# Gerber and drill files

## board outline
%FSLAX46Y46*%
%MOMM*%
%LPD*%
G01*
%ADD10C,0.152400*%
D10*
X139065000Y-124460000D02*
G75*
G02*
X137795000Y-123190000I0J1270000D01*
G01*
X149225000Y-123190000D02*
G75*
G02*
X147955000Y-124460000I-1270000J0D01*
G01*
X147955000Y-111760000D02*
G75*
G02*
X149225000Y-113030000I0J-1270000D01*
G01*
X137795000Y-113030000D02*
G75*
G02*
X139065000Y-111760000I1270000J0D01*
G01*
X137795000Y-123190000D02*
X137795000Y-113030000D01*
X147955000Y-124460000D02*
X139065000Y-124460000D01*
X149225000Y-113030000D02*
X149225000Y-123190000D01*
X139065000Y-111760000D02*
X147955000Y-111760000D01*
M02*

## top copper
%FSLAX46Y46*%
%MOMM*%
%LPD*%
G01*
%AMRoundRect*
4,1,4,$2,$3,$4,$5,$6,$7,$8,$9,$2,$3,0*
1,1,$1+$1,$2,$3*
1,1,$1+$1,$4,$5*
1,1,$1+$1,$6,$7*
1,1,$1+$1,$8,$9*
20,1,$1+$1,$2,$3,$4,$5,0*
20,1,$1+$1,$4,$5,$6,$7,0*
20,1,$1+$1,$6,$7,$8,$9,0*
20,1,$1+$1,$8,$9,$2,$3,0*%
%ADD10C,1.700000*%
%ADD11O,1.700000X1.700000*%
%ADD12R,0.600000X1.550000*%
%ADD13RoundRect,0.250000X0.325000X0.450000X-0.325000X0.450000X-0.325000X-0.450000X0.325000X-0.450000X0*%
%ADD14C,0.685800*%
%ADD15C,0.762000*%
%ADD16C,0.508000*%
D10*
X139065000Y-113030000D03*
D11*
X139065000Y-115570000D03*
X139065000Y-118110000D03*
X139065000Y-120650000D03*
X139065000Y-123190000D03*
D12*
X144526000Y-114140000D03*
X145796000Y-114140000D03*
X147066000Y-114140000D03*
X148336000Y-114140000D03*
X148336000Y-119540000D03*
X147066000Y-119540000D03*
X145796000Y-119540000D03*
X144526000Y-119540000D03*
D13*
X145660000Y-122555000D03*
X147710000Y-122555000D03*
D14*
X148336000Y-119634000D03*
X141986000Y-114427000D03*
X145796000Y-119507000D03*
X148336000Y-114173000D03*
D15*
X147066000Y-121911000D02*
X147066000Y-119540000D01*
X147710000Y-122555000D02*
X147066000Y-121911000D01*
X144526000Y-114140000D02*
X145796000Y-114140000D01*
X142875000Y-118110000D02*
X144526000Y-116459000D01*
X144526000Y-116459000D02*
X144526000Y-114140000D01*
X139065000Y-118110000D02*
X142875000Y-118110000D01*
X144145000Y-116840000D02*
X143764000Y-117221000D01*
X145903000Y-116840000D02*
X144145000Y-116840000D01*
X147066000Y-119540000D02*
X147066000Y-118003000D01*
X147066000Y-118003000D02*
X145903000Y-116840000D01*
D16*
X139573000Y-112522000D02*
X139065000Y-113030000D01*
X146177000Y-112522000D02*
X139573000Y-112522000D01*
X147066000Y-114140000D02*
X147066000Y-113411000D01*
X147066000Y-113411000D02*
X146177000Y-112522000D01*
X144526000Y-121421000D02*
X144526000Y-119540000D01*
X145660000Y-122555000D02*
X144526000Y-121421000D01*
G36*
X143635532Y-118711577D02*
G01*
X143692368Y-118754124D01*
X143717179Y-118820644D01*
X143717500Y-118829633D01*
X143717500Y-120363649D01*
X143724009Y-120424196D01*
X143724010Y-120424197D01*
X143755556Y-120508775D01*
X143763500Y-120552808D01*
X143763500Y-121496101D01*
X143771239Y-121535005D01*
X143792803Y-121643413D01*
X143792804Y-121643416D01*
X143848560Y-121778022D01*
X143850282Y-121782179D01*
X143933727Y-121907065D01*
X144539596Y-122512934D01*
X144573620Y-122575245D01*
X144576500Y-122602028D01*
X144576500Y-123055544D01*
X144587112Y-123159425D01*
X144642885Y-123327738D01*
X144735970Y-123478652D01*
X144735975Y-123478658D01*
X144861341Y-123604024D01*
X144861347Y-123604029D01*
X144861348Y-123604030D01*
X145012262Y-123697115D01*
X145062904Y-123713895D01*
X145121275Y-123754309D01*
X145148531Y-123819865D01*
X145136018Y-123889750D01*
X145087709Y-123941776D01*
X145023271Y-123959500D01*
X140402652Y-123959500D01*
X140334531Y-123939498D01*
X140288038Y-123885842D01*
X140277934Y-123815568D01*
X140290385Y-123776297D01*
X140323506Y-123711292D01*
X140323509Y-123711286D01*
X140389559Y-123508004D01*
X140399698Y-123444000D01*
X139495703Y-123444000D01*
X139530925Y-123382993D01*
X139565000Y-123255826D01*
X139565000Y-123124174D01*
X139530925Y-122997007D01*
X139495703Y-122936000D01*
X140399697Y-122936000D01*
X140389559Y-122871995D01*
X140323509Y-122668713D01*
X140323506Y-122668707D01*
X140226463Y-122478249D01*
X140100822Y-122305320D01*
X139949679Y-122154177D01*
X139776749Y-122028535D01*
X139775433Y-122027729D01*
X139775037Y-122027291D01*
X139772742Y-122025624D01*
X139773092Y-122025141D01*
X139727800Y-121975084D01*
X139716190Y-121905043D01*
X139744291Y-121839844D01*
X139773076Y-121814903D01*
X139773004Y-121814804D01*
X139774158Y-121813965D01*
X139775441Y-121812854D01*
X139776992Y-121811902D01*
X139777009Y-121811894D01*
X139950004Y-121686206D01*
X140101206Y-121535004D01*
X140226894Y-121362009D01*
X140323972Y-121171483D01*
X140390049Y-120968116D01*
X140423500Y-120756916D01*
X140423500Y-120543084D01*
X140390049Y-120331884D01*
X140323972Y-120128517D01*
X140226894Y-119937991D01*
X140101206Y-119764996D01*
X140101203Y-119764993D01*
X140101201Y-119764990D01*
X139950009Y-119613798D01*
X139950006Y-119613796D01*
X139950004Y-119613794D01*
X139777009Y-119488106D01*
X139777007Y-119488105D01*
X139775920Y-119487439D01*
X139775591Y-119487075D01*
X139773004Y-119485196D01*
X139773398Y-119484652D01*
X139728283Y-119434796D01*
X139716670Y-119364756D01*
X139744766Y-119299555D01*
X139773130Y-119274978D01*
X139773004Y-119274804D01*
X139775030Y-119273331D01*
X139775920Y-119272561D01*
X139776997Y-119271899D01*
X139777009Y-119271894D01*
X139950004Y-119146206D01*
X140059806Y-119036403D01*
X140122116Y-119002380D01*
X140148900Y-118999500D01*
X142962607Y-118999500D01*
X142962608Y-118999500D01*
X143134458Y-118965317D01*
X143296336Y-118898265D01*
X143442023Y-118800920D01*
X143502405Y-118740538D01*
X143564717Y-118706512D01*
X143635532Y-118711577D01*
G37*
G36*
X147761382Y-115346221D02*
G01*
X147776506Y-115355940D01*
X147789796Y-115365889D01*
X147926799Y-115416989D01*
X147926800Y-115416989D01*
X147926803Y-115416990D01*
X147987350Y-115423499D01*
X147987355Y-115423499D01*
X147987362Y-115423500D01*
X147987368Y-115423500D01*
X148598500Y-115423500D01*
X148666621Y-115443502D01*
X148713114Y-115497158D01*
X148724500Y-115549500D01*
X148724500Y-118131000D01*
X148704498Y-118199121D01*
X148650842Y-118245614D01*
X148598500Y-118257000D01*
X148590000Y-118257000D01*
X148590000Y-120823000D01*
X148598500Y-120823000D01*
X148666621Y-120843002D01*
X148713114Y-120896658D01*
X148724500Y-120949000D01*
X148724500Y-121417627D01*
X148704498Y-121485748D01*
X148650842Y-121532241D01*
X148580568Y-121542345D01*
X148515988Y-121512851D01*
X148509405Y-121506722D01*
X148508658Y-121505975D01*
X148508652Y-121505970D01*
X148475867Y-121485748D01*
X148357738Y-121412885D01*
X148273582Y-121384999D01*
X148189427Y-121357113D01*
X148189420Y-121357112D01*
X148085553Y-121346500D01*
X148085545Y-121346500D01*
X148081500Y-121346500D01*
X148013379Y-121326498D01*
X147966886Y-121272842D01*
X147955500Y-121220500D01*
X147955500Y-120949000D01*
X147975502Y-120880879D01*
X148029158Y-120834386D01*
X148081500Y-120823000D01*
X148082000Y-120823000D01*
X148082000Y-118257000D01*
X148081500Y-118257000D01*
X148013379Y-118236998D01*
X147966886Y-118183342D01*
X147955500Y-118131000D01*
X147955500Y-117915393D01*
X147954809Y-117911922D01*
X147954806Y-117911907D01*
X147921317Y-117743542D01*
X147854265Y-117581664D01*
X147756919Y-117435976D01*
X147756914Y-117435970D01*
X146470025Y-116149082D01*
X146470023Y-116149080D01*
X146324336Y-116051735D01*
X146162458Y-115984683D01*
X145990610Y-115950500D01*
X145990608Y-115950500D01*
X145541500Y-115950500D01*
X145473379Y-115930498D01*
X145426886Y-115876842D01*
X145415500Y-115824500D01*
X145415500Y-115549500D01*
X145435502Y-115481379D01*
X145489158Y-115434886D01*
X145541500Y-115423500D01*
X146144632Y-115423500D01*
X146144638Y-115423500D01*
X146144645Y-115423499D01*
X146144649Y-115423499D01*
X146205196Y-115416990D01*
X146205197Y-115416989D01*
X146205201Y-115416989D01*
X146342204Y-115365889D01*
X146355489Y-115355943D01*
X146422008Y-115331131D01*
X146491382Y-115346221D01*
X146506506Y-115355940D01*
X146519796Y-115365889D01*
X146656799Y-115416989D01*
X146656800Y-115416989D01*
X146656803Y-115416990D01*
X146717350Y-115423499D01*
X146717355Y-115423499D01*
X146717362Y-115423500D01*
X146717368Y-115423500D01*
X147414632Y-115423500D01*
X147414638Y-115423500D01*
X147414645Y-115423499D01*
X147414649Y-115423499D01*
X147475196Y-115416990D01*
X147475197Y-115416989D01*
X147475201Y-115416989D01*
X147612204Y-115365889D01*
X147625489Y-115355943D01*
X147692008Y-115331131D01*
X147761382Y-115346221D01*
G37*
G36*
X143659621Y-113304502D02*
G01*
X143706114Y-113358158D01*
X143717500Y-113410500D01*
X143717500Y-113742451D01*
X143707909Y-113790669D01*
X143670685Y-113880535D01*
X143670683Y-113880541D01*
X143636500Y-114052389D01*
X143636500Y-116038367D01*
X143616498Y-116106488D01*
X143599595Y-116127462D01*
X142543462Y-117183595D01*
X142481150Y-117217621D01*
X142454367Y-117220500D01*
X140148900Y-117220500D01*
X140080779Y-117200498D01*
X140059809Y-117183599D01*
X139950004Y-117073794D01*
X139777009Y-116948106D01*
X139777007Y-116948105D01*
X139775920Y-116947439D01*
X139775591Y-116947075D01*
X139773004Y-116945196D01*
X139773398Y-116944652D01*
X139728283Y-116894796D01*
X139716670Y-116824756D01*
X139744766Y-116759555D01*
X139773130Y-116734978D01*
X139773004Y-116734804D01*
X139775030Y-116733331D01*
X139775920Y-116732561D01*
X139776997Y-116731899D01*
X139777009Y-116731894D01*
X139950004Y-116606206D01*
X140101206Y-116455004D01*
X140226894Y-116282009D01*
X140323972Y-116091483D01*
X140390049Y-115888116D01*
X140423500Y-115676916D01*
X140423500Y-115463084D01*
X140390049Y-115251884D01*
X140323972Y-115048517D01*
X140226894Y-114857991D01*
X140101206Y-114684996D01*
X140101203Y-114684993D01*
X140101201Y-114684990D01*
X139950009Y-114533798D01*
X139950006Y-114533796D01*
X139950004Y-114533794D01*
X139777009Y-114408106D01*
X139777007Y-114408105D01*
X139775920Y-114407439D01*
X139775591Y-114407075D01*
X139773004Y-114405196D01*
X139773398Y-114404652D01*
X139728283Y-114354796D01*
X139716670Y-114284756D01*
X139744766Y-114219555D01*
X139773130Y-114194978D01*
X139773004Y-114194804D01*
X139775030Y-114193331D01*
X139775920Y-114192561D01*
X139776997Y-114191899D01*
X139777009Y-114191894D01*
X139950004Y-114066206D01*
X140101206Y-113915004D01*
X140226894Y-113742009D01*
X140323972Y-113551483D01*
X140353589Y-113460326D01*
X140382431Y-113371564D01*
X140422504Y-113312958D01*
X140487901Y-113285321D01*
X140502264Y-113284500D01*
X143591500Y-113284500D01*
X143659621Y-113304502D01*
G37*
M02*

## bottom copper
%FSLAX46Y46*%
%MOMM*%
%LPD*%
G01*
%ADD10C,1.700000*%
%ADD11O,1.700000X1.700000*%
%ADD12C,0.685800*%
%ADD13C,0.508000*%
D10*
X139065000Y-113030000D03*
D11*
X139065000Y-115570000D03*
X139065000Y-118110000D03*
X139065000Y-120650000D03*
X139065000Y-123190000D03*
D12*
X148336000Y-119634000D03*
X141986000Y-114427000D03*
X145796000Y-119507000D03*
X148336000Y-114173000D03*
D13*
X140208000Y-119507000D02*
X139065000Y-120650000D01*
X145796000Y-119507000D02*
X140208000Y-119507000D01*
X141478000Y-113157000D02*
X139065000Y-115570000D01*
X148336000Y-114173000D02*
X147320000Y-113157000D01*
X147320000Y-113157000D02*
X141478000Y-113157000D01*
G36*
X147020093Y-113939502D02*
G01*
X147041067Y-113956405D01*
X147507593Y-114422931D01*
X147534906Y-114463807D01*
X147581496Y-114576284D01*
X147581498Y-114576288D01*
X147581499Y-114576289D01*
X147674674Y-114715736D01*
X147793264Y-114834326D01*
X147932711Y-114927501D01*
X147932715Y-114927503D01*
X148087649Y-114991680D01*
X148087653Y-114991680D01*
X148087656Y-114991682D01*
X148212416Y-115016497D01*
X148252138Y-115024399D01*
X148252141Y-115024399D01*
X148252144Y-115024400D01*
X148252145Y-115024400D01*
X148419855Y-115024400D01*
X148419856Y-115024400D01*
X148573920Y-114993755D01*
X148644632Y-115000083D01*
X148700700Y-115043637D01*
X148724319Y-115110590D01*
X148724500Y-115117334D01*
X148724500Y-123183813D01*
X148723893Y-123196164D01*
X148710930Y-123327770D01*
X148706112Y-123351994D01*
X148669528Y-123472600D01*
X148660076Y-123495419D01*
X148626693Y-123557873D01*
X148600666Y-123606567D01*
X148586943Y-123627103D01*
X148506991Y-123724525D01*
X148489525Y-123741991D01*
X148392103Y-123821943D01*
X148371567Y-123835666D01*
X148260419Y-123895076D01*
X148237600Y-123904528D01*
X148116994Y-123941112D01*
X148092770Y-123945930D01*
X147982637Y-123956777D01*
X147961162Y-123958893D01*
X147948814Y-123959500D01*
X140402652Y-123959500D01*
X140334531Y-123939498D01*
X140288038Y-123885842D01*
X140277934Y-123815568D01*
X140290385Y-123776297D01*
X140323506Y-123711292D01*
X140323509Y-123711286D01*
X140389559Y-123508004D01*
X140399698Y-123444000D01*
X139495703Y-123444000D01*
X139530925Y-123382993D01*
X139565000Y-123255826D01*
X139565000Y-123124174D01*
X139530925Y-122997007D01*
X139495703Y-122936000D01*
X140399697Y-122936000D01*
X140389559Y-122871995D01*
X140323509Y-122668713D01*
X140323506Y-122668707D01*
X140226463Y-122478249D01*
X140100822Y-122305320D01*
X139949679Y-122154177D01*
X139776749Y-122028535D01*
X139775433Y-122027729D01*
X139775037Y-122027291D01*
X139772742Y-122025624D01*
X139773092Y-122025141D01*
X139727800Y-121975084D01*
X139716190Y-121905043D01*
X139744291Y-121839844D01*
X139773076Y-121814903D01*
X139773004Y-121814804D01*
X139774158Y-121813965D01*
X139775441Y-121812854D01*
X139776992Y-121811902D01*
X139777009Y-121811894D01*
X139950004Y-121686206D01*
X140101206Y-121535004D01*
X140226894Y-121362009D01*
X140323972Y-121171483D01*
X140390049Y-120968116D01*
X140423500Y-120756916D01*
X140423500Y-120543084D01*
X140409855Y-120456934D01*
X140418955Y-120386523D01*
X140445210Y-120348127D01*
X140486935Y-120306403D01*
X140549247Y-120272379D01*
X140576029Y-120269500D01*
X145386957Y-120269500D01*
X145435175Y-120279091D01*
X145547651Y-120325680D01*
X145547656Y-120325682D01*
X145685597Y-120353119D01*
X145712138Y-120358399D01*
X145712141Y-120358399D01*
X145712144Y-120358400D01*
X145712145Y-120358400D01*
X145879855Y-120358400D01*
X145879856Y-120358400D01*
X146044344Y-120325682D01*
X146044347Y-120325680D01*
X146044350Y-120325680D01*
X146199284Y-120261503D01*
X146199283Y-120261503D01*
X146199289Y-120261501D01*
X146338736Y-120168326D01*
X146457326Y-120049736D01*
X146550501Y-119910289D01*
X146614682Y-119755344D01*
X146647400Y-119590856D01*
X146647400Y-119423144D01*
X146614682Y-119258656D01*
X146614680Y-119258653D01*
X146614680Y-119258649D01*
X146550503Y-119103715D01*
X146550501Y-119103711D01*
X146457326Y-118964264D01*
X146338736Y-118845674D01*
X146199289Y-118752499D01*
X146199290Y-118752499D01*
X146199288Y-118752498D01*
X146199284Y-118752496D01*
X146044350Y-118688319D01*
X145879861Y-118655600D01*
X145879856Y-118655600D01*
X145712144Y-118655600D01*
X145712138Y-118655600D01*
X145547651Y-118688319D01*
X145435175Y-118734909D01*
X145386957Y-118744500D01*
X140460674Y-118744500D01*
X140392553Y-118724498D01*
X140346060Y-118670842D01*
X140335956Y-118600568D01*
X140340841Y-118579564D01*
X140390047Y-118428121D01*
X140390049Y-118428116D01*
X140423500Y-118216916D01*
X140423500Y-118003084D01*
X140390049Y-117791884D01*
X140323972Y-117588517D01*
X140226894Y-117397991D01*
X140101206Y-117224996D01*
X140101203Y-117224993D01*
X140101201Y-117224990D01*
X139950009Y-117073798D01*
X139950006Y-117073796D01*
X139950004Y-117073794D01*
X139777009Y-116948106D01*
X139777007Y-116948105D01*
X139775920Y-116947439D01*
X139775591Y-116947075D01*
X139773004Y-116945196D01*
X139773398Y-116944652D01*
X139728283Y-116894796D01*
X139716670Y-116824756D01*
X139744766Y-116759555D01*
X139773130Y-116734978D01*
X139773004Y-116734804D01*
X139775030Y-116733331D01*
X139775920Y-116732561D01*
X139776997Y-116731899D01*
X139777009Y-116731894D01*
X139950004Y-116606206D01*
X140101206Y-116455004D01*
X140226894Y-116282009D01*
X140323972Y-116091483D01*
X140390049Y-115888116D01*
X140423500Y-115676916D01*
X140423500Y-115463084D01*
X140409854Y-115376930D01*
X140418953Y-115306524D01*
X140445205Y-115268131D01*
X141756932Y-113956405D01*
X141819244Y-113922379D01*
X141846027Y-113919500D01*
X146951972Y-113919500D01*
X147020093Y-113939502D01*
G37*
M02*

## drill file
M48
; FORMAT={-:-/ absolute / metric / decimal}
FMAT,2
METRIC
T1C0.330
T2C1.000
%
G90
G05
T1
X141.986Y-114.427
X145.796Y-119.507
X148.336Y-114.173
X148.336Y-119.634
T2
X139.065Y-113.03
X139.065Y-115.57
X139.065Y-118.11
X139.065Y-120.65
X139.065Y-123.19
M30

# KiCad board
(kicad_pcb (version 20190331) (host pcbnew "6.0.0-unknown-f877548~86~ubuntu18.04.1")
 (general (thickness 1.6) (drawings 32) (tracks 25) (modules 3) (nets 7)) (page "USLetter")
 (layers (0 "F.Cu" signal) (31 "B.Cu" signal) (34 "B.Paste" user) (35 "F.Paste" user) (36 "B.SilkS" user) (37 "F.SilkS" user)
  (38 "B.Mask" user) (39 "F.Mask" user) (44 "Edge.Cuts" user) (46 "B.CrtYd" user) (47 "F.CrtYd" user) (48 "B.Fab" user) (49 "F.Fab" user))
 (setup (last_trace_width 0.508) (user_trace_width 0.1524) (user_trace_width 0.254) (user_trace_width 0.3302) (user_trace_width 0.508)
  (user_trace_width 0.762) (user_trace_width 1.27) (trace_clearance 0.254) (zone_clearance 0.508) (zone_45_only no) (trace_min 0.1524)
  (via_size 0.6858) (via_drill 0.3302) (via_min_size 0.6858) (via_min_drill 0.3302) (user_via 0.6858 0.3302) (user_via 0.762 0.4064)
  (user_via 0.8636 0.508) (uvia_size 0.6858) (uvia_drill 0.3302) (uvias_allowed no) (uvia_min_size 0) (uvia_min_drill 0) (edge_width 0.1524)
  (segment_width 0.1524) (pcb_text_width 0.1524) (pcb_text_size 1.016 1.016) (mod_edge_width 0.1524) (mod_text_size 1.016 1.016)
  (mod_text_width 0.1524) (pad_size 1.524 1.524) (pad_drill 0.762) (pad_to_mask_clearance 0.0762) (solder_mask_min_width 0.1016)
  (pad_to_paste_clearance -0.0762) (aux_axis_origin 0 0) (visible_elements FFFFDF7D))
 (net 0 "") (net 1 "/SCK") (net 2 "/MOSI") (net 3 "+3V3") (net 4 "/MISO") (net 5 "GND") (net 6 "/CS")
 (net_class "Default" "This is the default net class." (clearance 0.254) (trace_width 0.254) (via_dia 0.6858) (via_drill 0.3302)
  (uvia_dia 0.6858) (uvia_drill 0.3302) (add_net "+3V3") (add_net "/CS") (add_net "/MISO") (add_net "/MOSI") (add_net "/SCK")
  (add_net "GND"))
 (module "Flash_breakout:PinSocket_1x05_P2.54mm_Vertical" (layer "F.Cu") (at 139.065 113.03)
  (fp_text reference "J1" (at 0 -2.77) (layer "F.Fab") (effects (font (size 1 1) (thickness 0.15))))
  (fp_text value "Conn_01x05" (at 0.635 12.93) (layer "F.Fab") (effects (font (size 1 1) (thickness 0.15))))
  (pad "1" thru_hole circle (at 0 0) (size 1.7 1.7) (drill 1) (layers *.Cu *.Mask) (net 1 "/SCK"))
  (pad "2" thru_hole oval (at 0 2.54) (size 1.7 1.7) (drill 1) (layers *.Cu *.Mask) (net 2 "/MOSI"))
  (pad "3" thru_hole oval (at 0 5.08) (size 1.7 1.7) (drill 1) (layers *.Cu *.Mask) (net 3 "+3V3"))
  (pad "4" thru_hole oval (at 0 7.62) (size 1.7 1.7) (drill 1) (layers *.Cu *.Mask) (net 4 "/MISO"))
  (pad "5" thru_hole oval (at 0 10.16) (size 1.7 1.7) (drill 1) (layers *.Cu *.Mask) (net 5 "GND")))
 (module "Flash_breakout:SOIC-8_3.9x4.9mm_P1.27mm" (layer "F.Cu") (at 146.431 116.84 90)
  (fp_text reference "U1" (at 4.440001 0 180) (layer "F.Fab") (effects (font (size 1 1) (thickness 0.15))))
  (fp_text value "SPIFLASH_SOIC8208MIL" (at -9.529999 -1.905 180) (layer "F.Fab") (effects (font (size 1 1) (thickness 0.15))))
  (pad "8" smd rect (at 2.7 -1.905 90) (size 1.55 0.6) (layers "F.Cu" "F.Paste" "F.Mask") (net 3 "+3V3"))
  (pad "7" smd rect (at 2.7 -0.635 90) (size 1.55 0.6) (layers "F.Cu" "F.Paste" "F.Mask") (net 3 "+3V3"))
  (pad "6" smd rect (at 2.7 0.635 90) (size 1.55 0.6) (layers "F.Cu" "F.Paste" "F.Mask") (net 1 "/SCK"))
  (pad "5" smd rect (at 2.7 1.905 90) (size 1.55 0.6) (layers "F.Cu" "F.Paste" "F.Mask") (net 2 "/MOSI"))
  (pad "4" smd rect (at -2.7 1.905 90) (size 1.55 0.6) (layers "F.Cu" "F.Paste" "F.Mask") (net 5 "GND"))
  (pad "3" smd rect (at -2.7 0.635 90) (size 1.55 0.6) (layers "F.Cu" "F.Paste" "F.Mask") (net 3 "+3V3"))
  (pad "2" smd rect (at -2.7 -0.635 90) (size 1.55 0.6) (layers "F.Cu" "F.Paste" "F.Mask") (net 4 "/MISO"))
  (pad "1" smd rect (at -2.7 -1.905 90) (size 1.55 0.6) (layers "F.Cu" "F.Paste" "F.Mask") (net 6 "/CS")))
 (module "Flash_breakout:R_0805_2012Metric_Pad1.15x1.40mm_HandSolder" (layer "F.Cu") (at 146.685 122.555 180)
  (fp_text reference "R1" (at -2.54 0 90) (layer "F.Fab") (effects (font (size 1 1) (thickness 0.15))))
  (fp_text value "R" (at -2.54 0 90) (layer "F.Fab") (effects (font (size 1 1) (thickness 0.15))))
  (pad "2" smd roundrect (at 1.025 0 180) (size 1.15 1.4) (layers "F.Cu" "F.Paste" "F.Mask") (roundrect_rratio 0.217391) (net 6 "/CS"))
  (pad "1" smd roundrect (at -1.025 0 180) (size 1.15 1.4) (layers "F.Cu" "F.Paste" "F.Mask") (roundrect_rratio 0.217391) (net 3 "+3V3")))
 (gr_arc (start 139.065 123.19) (end 137.795 123.19) (angle -90) (layer "Edge.Cuts") (width 0.1524))
 (gr_arc (start 147.955 123.19) (end 147.955 124.46) (angle -90) (layer "Edge.Cuts") (width 0.1524))
 (gr_arc (start 147.955 113.03) (end 149.225 113.03) (angle -90) (layer "Edge.Cuts") (width 0.1524))
 (gr_arc (start 139.065 113.03) (end 139.065 111.76) (angle -90) (layer "Edge.Cuts") (width 0.1524))
 (gr_line (start 137.795 123.19) (end 137.795 113.03) (layer "Edge.Cuts") (width 0.1524))
 (gr_line (start 147.955 124.46) (end 139.065 124.46) (layer "Edge.Cuts") (width 0.1524))
 (gr_line (start 149.225 113.03) (end 149.225 123.19) (layer "Edge.Cuts") (width 0.1524))
 (gr_line (start 139.065 111.76) (end 147.955 111.76) (layer "Edge.Cuts") (width 0.1524))
 (via (at 148.336 119.634) (size 0.6858) (drill 0.3302) (layers "F.Cu" "B.Cu") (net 5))
 (via (at 141.986 114.427) (size 0.6858) (drill 0.3302) (layers "F.Cu" "B.Cu") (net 5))
 (via (at 145.796 119.507) (size 0.6858) (drill 0.3302) (layers "F.Cu" "B.Cu") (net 4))
 (via (at 148.336 114.173) (size 0.6858) (drill 0.3302) (layers "F.Cu" "B.Cu") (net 2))
 (segment (start 147.066 121.911) (end 147.066 119.54) (width 0.762) (layer "F.Cu") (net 3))
 (segment (start 147.71 122.555) (end 147.066 121.911) (width 0.762) (layer "F.Cu") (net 3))
 (segment (start 144.526 114.14) (end 145.796 114.14) (width 0.762) (layer "F.Cu") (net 3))
 (segment (start 142.875 118.11) (end 144.526 116.459) (width 0.762) (layer "F.Cu") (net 3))
 (segment (start 144.526 116.459) (end 144.526 114.14) (width 0.762) (layer "F.Cu") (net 3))
 (segment (start 139.065 118.11) (end 142.875 118.11) (width 0.762) (layer "F.Cu") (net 3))
 (segment (start 144.145 116.84) (end 143.764 117.221) (width 0.762) (layer "F.Cu") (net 3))
 (segment (start 145.903 116.84) (end 144.145 116.84) (width 0.762) (layer "F.Cu") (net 3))
 (segment (start 147.066 119.54) (end 147.066 118.003) (width 0.762) (layer "F.Cu") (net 3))
 (segment (start 147.066 118.003) (end 145.903 116.84) (width 0.762) (layer "F.Cu") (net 3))
 (segment (start 140.208 119.507) (end 139.065 120.65) (width 0.508) (layer "B.Cu") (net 4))
 (segment (start 145.796 119.507) (end 140.208 119.507) (width 0.508) (layer "B.Cu") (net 4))
 (segment (start 141.478 113.157) (end 139.065 115.57) (width 0.508) (layer "B.Cu") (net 2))
 (segment (start 148.336 114.173) (end 147.32 113.157) (width 0.508) (layer "B.Cu") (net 2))
 (segment (start 147.32 113.157) (end 141.478 113.157) (width 0.508) (layer "B.Cu") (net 2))
 (segment (start 139.573 112.522) (end 139.065 113.03) (width 0.508) (layer "F.Cu") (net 1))
 (segment (start 146.177 112.522) (end 139.573 112.522) (width 0.508) (layer "F.Cu") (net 1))
 (segment (start 147.066 114.14) (end 147.066 113.411) (width 0.508) (layer "F.Cu") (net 1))
 (segment (start 147.066 113.411) (end 146.177 112.522) (width 0.508) (layer "F.Cu") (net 1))
 (segment (start 144.526 121.421) (end 144.526 119.54) (width 0.508) (layer "F.Cu") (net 6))
 (segment (start 145.66 122.555) (end 144.526 121.421) (width 0.508) (layer "F.Cu") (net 6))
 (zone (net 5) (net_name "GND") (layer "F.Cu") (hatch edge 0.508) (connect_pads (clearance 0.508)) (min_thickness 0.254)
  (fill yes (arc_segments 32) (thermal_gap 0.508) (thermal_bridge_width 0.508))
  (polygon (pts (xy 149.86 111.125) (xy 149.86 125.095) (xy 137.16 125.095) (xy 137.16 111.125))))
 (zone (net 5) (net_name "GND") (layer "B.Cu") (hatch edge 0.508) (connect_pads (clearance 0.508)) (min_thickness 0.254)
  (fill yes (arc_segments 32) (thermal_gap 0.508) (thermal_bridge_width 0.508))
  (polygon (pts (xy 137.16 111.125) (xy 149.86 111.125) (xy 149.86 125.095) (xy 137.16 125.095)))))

